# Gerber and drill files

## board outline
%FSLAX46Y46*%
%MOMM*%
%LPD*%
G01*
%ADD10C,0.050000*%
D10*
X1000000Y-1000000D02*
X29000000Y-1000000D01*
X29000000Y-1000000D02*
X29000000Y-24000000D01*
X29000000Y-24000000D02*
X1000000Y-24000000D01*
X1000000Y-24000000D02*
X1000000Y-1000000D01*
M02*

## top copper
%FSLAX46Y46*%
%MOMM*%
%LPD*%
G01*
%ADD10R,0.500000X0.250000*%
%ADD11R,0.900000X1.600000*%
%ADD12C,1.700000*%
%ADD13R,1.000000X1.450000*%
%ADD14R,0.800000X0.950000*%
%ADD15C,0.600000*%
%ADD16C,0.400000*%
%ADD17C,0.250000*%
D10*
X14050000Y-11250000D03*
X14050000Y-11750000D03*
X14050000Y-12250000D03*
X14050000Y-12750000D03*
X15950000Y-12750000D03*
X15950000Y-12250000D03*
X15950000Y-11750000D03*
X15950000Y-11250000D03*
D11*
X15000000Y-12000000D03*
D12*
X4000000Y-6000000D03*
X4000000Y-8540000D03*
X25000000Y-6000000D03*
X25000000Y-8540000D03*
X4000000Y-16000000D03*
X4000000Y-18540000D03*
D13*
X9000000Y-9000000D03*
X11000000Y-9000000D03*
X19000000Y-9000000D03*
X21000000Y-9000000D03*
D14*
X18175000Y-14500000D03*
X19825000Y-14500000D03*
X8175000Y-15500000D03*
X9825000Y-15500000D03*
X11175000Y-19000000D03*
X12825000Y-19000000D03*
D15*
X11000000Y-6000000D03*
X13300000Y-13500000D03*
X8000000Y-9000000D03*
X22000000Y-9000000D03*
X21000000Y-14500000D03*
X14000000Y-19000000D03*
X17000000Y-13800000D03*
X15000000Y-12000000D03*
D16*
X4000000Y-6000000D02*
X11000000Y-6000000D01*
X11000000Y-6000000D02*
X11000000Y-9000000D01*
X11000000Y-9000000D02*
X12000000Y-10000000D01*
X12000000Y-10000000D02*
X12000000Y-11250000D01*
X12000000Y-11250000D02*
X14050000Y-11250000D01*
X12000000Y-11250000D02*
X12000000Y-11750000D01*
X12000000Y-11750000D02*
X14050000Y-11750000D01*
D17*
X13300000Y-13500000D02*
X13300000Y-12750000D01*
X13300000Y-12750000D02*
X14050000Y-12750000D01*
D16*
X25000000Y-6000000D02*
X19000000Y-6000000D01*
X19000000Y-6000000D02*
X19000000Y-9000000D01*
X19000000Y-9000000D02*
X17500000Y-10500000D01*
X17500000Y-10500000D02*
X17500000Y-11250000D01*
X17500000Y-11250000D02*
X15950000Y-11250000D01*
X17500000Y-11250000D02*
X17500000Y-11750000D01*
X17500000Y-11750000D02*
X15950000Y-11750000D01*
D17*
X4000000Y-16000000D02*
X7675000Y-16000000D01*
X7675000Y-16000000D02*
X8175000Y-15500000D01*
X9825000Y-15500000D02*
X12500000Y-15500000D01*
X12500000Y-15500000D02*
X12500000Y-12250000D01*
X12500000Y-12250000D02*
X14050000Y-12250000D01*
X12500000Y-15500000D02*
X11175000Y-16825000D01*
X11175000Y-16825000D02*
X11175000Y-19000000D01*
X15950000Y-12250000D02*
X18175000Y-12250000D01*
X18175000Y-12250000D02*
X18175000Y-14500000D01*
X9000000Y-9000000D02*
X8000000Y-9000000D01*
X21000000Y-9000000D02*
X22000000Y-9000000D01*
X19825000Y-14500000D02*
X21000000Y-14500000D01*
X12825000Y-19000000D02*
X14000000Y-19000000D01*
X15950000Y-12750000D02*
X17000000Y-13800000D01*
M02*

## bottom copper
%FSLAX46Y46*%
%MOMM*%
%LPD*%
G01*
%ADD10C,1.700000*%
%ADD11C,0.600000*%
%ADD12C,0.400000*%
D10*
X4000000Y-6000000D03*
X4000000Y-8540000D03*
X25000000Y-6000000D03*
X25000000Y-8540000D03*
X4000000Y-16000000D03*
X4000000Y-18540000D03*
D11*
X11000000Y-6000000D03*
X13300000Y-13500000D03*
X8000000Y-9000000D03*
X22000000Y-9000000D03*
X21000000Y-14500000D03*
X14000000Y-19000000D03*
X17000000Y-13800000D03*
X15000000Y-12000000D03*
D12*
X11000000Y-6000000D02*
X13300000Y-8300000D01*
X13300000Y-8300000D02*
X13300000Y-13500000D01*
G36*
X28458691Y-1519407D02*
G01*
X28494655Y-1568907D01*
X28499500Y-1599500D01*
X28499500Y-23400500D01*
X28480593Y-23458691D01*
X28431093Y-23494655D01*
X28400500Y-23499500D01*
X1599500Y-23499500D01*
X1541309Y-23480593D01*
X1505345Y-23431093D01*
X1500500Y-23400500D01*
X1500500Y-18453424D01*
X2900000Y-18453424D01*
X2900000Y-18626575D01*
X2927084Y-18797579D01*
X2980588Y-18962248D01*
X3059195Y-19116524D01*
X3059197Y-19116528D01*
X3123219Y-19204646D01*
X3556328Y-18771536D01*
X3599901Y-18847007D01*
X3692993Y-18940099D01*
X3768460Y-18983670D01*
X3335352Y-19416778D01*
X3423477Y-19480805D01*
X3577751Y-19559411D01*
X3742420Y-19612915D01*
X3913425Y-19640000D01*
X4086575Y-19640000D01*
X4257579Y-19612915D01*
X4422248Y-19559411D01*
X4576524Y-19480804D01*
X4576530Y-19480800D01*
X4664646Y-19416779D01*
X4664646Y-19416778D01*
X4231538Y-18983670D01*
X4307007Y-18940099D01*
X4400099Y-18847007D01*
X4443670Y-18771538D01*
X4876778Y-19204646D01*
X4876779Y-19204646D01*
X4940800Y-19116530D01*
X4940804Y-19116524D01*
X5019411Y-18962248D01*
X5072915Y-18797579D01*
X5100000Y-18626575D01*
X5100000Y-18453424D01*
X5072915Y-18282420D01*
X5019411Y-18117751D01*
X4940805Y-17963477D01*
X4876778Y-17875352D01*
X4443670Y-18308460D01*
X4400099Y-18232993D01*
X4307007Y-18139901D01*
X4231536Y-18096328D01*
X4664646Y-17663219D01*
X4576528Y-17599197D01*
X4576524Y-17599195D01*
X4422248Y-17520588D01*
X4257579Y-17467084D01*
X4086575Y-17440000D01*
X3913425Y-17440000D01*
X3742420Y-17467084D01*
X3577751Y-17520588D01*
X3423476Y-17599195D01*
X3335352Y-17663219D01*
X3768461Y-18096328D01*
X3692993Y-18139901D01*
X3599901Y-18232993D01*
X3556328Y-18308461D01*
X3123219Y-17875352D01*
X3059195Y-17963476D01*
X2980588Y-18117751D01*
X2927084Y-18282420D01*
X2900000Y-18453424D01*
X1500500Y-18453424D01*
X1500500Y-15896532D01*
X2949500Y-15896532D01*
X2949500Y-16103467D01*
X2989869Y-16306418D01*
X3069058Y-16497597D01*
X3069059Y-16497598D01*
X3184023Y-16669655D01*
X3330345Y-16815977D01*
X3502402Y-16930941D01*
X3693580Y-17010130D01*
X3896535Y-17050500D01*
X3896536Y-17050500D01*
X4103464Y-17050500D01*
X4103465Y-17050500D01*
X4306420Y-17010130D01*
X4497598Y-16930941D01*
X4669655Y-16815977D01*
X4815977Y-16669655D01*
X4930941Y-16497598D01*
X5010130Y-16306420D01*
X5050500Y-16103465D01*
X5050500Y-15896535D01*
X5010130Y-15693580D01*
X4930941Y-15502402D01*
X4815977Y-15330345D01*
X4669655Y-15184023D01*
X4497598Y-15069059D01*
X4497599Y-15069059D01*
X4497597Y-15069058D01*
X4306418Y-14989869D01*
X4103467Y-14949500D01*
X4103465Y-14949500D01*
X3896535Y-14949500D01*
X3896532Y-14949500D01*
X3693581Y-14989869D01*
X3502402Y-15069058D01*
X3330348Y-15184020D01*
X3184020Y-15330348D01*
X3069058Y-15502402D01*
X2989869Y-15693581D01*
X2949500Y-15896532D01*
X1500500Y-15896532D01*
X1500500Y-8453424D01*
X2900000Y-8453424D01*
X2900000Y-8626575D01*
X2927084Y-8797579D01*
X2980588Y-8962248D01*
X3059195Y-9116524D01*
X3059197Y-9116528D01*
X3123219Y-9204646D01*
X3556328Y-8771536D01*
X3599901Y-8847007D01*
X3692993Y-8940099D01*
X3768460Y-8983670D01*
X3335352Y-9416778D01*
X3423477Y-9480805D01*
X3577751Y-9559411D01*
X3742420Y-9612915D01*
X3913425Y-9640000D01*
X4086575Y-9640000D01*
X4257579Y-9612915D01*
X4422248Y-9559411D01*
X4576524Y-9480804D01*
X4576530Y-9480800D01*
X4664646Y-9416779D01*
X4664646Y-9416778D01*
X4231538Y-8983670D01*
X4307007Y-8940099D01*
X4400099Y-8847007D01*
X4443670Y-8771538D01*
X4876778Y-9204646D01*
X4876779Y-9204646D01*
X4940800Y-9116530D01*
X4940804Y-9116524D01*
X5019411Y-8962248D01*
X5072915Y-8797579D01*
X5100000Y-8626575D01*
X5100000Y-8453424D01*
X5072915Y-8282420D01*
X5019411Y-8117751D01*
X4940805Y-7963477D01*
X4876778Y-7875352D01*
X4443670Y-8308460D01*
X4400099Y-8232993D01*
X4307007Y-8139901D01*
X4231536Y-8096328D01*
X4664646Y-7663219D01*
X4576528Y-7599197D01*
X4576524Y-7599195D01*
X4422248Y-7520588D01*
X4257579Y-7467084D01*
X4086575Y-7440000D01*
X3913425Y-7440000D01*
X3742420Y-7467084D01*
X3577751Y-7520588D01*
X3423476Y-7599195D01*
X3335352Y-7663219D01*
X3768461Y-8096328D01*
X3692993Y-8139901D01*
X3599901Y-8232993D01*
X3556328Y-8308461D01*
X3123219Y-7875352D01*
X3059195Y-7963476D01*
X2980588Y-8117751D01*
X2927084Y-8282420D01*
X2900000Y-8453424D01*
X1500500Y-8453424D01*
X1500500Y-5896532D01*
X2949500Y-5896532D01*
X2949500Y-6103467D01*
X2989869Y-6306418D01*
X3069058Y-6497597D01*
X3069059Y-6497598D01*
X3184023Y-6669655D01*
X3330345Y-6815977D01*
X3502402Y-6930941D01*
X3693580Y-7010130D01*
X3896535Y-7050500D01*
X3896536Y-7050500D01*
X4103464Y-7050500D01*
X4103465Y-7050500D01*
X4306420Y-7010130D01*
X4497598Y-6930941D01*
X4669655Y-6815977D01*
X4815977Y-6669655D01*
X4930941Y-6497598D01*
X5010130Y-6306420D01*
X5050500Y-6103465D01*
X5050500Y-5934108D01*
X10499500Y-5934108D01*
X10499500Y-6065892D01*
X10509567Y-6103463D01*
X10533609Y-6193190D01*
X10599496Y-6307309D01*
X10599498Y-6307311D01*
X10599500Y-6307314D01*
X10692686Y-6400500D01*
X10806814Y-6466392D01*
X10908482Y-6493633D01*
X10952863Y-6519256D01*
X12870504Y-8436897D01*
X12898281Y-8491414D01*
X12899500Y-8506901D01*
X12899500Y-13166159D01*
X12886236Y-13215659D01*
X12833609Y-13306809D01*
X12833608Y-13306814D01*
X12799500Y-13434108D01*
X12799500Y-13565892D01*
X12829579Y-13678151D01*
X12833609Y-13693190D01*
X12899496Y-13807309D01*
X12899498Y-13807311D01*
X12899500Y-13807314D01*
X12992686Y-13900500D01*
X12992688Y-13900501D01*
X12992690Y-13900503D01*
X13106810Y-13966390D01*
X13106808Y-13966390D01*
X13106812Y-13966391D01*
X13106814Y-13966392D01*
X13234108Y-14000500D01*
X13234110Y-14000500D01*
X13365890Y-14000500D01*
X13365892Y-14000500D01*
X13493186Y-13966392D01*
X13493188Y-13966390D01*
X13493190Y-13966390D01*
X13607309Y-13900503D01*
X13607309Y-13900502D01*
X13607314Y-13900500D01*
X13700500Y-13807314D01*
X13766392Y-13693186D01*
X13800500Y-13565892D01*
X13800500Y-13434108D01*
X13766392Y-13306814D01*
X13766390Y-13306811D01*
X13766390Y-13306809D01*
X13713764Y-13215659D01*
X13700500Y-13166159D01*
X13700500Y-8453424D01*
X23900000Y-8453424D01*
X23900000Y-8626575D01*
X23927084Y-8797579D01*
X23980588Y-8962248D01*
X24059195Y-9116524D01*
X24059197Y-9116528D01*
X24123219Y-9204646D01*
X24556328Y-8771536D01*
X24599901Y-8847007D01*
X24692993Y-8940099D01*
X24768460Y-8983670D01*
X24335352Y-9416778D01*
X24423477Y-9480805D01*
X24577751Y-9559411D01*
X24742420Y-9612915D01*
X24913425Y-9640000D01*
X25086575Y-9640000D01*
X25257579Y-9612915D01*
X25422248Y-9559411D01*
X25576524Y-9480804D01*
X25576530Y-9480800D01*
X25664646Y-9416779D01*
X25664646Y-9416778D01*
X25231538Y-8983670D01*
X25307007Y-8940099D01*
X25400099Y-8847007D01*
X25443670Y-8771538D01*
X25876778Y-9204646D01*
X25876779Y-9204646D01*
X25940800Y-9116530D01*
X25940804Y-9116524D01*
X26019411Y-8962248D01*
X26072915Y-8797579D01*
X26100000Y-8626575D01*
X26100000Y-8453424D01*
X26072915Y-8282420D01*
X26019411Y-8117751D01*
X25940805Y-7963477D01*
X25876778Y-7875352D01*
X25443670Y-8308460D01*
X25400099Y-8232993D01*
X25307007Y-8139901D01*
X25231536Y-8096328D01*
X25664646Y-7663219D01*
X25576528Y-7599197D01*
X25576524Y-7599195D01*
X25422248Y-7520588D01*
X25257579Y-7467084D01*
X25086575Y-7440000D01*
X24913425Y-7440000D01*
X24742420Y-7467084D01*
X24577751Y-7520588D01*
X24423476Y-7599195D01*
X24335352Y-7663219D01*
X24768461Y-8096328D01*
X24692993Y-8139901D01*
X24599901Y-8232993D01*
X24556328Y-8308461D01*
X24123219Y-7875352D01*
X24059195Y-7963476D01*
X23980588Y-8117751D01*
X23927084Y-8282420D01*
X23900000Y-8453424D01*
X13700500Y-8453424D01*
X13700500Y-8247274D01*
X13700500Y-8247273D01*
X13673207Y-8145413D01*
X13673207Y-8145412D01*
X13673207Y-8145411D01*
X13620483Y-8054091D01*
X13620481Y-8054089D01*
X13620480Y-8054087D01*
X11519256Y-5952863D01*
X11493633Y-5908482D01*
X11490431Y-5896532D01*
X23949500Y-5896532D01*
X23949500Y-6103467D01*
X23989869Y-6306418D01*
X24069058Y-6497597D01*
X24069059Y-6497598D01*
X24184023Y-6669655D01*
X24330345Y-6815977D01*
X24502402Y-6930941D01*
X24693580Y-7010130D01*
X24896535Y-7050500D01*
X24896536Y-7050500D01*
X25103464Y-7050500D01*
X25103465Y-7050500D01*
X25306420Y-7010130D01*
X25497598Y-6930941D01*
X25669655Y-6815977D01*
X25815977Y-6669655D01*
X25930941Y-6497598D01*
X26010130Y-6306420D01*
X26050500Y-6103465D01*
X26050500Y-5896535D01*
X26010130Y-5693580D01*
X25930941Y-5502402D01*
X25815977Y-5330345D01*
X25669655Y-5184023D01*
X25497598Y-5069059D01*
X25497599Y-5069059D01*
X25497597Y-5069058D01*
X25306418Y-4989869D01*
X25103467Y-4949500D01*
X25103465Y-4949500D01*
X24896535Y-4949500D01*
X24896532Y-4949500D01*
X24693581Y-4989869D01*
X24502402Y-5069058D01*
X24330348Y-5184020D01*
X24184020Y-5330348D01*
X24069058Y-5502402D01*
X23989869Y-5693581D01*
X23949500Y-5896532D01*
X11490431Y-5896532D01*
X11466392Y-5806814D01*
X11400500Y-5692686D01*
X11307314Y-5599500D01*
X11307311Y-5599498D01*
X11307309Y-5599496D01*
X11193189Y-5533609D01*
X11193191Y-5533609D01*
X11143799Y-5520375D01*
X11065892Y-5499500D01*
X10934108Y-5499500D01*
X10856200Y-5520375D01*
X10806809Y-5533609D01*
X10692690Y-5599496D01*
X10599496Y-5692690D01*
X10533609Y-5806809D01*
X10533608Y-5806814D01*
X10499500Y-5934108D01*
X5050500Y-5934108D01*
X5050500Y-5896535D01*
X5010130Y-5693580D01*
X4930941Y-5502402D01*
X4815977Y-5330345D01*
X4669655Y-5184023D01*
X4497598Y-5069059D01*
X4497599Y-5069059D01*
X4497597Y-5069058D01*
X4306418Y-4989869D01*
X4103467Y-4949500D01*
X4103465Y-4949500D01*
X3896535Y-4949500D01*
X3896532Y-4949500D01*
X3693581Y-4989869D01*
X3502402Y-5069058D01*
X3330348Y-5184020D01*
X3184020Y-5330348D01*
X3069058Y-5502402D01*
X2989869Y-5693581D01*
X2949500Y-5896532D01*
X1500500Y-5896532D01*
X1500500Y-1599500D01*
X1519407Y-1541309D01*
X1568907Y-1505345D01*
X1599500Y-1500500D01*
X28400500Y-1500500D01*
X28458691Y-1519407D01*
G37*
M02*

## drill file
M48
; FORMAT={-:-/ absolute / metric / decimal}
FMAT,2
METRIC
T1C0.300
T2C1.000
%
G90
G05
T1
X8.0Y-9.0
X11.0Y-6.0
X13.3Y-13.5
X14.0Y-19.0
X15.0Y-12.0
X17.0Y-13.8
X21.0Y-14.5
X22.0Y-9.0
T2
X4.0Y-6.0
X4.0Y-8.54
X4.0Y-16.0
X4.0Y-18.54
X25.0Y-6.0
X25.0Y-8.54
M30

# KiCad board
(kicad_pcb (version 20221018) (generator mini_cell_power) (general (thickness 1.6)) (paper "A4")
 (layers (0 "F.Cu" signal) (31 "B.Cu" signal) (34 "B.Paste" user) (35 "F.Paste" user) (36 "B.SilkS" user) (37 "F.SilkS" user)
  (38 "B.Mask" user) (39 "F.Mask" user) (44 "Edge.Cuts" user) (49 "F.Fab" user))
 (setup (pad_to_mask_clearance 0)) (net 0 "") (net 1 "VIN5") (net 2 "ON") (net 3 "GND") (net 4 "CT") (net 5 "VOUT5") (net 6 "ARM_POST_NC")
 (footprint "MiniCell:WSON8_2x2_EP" (layer "F.Cu") (at 15 12)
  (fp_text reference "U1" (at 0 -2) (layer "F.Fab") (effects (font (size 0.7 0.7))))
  (pad "1" smd rect (at -0.95 -0.75) (size 0.5 0.25) (layers "F.Cu" "F.Paste" "F.Mask") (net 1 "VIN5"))
  (pad "2" smd rect (at -0.95 -0.25) (size 0.5 0.25) (layers "F.Cu" "F.Paste" "F.Mask") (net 1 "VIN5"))
  (pad "3" smd rect (at -0.95 0.25) (size 0.5 0.25) (layers "F.Cu" "F.Paste" "F.Mask") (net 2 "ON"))
  (pad "4" smd rect (at -0.95 0.75) (size 0.5 0.25) (layers "F.Cu" "F.Paste" "F.Mask") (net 1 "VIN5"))
  (pad "5" smd rect (at 0.95 0.75) (size 0.5 0.25) (layers "F.Cu" "F.Paste" "F.Mask") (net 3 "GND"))
  (pad "6" smd rect (at 0.95 0.25) (size 0.5 0.25) (layers "F.Cu" "F.Paste" "F.Mask") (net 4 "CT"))
  (pad "7" smd rect (at 0.95 -0.25) (size 0.5 0.25) (layers "F.Cu" "F.Paste" "F.Mask") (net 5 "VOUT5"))
  (pad "8" smd rect (at 0.95 -0.75) (size 0.5 0.25) (layers "F.Cu" "F.Paste" "F.Mask") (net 5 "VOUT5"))
  (pad "9" smd rect (at 0 0) (size 0.9 1.6) (layers "F.Cu" "F.Paste" "F.Mask") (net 3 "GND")))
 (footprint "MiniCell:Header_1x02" (layer "F.Cu") (at 4 6)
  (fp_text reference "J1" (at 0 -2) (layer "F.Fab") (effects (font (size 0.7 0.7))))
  (pad "1" thru_hole circle (at 0 0.0) (size 1.7 1.7) (drill 1) (layers "*.Cu" "*.Mask") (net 1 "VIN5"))
  (pad "2" thru_hole circle (at 0 2.54) (size 1.7 1.7) (drill 1) (layers "*.Cu" "*.Mask") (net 3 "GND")))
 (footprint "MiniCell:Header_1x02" (layer "F.Cu") (at 25 6)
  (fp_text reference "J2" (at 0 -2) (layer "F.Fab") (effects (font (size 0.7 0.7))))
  (pad "1" thru_hole circle (at 0 0.0) (size 1.7 1.7) (drill 1) (layers "*.Cu" "*.Mask") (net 5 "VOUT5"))
  (pad "2" thru_hole circle (at 0 2.54) (size 1.7 1.7) (drill 1) (layers "*.Cu" "*.Mask") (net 3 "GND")))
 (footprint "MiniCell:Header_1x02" (layer "F.Cu") (at 4 16)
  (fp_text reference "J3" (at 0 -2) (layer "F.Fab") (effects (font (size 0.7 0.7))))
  (pad "1" thru_hole circle (at 0 0.0) (size 1.7 1.7) (drill 1) (layers "*.Cu" "*.Mask") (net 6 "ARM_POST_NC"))
  (pad "2" thru_hole circle (at 0 2.54) (size 1.7 1.7) (drill 1) (layers "*.Cu" "*.Mask") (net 3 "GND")))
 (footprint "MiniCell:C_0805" (layer "F.Cu") (at 10 9)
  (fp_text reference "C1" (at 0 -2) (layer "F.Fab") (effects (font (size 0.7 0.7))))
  (pad "1" smd rect (at -1 0) (size 1 1.45) (layers "F.Cu" "F.Paste" "F.Mask") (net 3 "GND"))
  (pad "2" smd rect (at 1 0) (size 1 1.45) (layers "F.Cu" "F.Paste" "F.Mask") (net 1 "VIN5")))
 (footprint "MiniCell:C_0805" (layer "F.Cu") (at 20 9)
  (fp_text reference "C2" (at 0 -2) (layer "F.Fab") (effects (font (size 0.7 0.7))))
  (pad "1" smd rect (at -1 0) (size 1 1.45) (layers "F.Cu" "F.Paste" "F.Mask") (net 5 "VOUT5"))
  (pad "2" smd rect (at 1 0) (size 1 1.45) (layers "F.Cu" "F.Paste" "F.Mask") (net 3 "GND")))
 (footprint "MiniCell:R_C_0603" (layer "F.Cu") (at 19 14.5)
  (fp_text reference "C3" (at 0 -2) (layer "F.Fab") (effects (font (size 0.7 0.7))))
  (pad "1" smd rect (at -0.825 0) (size 0.8 0.95) (layers "F.Cu" "F.Paste" "F.Mask") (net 4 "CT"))
  (pad "2" smd rect (at 0.825 0) (size 0.8 0.95) (layers "F.Cu" "F.Paste" "F.Mask") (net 3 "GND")))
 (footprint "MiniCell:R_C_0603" (layer "F.Cu") (at 9 15.5)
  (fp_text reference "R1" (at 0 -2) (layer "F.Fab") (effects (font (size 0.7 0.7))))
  (pad "1" smd rect (at -0.825 0) (size 0.8 0.95) (layers "F.Cu" "F.Paste" "F.Mask") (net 6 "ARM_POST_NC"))
  (pad "2" smd rect (at 0.825 0) (size 0.8 0.95) (layers "F.Cu" "F.Paste" "F.Mask") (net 2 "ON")))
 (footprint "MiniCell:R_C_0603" (layer "F.Cu") (at 12 19)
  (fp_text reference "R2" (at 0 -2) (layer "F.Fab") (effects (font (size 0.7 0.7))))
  (pad "1" smd rect (at -0.825 0) (size 0.8 0.95) (layers "F.Cu" "F.Paste" "F.Mask") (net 2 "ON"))
  (pad "2" smd rect (at 0.825 0) (size 0.8 0.95) (layers "F.Cu" "F.Paste" "F.Mask") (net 3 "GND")))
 (segment (start 4 6) (end 11 6) (width 0.4) (layer "F.Cu") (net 1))
 (segment (start 11 6) (end 11 9) (width 0.4) (layer "F.Cu") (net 1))
 (segment (start 11 9) (end 12 10) (width 0.4) (layer "F.Cu") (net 1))
 (segment (start 12 10) (end 12 11.25) (width 0.4) (layer "F.Cu") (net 1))
 (segment (start 12 11.25) (end 14.05 11.25) (width 0.4) (layer "F.Cu") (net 1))
 (segment (start 12 11.25) (end 12 11.75) (width 0.4) (layer "F.Cu") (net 1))
 (segment (start 12 11.75) (end 14.05 11.75) (width 0.4) (layer "F.Cu") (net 1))
 (via (at 11 6) (size .6) (drill .3) (layers "F.Cu" "B.Cu") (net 1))
 (via (at 13.3 13.5) (size .6) (drill .3) (layers "F.Cu" "B.Cu") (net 1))
 (segment (start 11 6) (end 13.3 8.3) (width 0.4) (layer "B.Cu") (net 1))
 (segment (start 13.3 8.3) (end 13.3 13.5) (width 0.4) (layer "B.Cu") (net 1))
 (segment (start 13.3 13.5) (end 13.3 12.75) (width 0.25) (layer "F.Cu") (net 1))
 (segment (start 13.3 12.75) (end 14.05 12.75) (width 0.25) (layer "F.Cu") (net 1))
 (segment (start 25 6) (end 19 6) (width 0.4) (layer "F.Cu") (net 5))
 (segment (start 19 6) (end 19 9) (width 0.4) (layer "F.Cu") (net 5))
 (segment (start 19 9) (end 17.5 10.5) (width 0.4) (layer "F.Cu") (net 5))
 (segment (start 17.5 10.5) (end 17.5 11.25) (width 0.4) (layer "F.Cu") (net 5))
 (segment (start 17.5 11.25) (end 15.95 11.25) (width 0.4) (layer "F.Cu") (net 5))
 (segment (start 17.5 11.25) (end 17.5 11.75) (width 0.4) (layer "F.Cu") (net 5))
 (segment (start 17.5 11.75) (end 15.95 11.75) (width 0.4) (layer "F.Cu") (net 5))
 (segment (start 4 16) (end 7.675 16) (width 0.25) (layer "F.Cu") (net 6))
 (segment (start 7.675 16) (end 8.175 15.5) (width 0.25) (layer "F.Cu") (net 6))
 (segment (start 9.825 15.5) (end 12.5 15.5) (width 0.25) (layer "F.Cu") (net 2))
 (segment (start 12.5 15.5) (end 12.5 12.25) (width 0.25) (layer "F.Cu") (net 2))
 (segment (start 12.5 12.25) (end 14.05 12.25) (width 0.25) (layer "F.Cu") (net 2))
 (segment (start 12.5 15.5) (end 11.175 16.825) (width 0.25) (layer "F.Cu") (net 2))
 (segment (start 11.175 16.825) (end 11.175 19) (width 0.25) (layer "F.Cu") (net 2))
 (segment (start 15.95 12.25) (end 18.175 12.25) (width 0.25) (layer "F.Cu") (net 4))
 (segment (start 18.175 12.25) (end 18.175 14.5) (width 0.25) (layer "F.Cu") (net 4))
 (segment (start 9 9) (end 8 9) (width 0.25) (layer "F.Cu") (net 3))
 (via (at 8 9) (size .6) (drill .3) (layers "F.Cu" "B.Cu") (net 3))
 (segment (start 21 9) (end 22 9) (width 0.25) (layer "F.Cu") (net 3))
 (via (at 22 9) (size .6) (drill .3) (layers "F.Cu" "B.Cu") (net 3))
 (segment (start 19.825 14.5) (end 21 14.5) (width 0.25) (layer "F.Cu") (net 3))
 (via (at 21 14.5) (size .6) (drill .3) (layers "F.Cu" "B.Cu") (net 3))
 (segment (start 12.825 19) (end 14 19) (width 0.25) (layer "F.Cu") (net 3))
 (via (at 14 19) (size .6) (drill .3) (layers "F.Cu" "B.Cu") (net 3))
 (segment (start 15.95 12.75) (end 17 13.8) (width 0.25) (layer "F.Cu") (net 3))
 (via (at 17 13.8) (size .6) (drill .3) (layers "F.Cu" "B.Cu") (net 3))
 (via (at 15 12) (size .6) (drill .3) (layers "F.Cu" "B.Cu") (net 3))
 (gr_line (start 1 1) (end 29 1) (layer "Edge.Cuts") (width .05))
 (gr_line (start 29 1) (end 29 24) (layer "Edge.Cuts") (width .05))
 (gr_line (start 29 24) (end 1 24) (layer "Edge.Cuts") (width .05))
 (gr_line (start 1 24) (end 1 1) (layer "Edge.Cuts") (width .05))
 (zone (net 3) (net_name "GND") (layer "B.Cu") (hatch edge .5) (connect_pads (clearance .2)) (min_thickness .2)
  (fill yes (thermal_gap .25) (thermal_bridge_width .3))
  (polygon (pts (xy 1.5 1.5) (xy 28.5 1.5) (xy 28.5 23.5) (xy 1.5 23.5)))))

